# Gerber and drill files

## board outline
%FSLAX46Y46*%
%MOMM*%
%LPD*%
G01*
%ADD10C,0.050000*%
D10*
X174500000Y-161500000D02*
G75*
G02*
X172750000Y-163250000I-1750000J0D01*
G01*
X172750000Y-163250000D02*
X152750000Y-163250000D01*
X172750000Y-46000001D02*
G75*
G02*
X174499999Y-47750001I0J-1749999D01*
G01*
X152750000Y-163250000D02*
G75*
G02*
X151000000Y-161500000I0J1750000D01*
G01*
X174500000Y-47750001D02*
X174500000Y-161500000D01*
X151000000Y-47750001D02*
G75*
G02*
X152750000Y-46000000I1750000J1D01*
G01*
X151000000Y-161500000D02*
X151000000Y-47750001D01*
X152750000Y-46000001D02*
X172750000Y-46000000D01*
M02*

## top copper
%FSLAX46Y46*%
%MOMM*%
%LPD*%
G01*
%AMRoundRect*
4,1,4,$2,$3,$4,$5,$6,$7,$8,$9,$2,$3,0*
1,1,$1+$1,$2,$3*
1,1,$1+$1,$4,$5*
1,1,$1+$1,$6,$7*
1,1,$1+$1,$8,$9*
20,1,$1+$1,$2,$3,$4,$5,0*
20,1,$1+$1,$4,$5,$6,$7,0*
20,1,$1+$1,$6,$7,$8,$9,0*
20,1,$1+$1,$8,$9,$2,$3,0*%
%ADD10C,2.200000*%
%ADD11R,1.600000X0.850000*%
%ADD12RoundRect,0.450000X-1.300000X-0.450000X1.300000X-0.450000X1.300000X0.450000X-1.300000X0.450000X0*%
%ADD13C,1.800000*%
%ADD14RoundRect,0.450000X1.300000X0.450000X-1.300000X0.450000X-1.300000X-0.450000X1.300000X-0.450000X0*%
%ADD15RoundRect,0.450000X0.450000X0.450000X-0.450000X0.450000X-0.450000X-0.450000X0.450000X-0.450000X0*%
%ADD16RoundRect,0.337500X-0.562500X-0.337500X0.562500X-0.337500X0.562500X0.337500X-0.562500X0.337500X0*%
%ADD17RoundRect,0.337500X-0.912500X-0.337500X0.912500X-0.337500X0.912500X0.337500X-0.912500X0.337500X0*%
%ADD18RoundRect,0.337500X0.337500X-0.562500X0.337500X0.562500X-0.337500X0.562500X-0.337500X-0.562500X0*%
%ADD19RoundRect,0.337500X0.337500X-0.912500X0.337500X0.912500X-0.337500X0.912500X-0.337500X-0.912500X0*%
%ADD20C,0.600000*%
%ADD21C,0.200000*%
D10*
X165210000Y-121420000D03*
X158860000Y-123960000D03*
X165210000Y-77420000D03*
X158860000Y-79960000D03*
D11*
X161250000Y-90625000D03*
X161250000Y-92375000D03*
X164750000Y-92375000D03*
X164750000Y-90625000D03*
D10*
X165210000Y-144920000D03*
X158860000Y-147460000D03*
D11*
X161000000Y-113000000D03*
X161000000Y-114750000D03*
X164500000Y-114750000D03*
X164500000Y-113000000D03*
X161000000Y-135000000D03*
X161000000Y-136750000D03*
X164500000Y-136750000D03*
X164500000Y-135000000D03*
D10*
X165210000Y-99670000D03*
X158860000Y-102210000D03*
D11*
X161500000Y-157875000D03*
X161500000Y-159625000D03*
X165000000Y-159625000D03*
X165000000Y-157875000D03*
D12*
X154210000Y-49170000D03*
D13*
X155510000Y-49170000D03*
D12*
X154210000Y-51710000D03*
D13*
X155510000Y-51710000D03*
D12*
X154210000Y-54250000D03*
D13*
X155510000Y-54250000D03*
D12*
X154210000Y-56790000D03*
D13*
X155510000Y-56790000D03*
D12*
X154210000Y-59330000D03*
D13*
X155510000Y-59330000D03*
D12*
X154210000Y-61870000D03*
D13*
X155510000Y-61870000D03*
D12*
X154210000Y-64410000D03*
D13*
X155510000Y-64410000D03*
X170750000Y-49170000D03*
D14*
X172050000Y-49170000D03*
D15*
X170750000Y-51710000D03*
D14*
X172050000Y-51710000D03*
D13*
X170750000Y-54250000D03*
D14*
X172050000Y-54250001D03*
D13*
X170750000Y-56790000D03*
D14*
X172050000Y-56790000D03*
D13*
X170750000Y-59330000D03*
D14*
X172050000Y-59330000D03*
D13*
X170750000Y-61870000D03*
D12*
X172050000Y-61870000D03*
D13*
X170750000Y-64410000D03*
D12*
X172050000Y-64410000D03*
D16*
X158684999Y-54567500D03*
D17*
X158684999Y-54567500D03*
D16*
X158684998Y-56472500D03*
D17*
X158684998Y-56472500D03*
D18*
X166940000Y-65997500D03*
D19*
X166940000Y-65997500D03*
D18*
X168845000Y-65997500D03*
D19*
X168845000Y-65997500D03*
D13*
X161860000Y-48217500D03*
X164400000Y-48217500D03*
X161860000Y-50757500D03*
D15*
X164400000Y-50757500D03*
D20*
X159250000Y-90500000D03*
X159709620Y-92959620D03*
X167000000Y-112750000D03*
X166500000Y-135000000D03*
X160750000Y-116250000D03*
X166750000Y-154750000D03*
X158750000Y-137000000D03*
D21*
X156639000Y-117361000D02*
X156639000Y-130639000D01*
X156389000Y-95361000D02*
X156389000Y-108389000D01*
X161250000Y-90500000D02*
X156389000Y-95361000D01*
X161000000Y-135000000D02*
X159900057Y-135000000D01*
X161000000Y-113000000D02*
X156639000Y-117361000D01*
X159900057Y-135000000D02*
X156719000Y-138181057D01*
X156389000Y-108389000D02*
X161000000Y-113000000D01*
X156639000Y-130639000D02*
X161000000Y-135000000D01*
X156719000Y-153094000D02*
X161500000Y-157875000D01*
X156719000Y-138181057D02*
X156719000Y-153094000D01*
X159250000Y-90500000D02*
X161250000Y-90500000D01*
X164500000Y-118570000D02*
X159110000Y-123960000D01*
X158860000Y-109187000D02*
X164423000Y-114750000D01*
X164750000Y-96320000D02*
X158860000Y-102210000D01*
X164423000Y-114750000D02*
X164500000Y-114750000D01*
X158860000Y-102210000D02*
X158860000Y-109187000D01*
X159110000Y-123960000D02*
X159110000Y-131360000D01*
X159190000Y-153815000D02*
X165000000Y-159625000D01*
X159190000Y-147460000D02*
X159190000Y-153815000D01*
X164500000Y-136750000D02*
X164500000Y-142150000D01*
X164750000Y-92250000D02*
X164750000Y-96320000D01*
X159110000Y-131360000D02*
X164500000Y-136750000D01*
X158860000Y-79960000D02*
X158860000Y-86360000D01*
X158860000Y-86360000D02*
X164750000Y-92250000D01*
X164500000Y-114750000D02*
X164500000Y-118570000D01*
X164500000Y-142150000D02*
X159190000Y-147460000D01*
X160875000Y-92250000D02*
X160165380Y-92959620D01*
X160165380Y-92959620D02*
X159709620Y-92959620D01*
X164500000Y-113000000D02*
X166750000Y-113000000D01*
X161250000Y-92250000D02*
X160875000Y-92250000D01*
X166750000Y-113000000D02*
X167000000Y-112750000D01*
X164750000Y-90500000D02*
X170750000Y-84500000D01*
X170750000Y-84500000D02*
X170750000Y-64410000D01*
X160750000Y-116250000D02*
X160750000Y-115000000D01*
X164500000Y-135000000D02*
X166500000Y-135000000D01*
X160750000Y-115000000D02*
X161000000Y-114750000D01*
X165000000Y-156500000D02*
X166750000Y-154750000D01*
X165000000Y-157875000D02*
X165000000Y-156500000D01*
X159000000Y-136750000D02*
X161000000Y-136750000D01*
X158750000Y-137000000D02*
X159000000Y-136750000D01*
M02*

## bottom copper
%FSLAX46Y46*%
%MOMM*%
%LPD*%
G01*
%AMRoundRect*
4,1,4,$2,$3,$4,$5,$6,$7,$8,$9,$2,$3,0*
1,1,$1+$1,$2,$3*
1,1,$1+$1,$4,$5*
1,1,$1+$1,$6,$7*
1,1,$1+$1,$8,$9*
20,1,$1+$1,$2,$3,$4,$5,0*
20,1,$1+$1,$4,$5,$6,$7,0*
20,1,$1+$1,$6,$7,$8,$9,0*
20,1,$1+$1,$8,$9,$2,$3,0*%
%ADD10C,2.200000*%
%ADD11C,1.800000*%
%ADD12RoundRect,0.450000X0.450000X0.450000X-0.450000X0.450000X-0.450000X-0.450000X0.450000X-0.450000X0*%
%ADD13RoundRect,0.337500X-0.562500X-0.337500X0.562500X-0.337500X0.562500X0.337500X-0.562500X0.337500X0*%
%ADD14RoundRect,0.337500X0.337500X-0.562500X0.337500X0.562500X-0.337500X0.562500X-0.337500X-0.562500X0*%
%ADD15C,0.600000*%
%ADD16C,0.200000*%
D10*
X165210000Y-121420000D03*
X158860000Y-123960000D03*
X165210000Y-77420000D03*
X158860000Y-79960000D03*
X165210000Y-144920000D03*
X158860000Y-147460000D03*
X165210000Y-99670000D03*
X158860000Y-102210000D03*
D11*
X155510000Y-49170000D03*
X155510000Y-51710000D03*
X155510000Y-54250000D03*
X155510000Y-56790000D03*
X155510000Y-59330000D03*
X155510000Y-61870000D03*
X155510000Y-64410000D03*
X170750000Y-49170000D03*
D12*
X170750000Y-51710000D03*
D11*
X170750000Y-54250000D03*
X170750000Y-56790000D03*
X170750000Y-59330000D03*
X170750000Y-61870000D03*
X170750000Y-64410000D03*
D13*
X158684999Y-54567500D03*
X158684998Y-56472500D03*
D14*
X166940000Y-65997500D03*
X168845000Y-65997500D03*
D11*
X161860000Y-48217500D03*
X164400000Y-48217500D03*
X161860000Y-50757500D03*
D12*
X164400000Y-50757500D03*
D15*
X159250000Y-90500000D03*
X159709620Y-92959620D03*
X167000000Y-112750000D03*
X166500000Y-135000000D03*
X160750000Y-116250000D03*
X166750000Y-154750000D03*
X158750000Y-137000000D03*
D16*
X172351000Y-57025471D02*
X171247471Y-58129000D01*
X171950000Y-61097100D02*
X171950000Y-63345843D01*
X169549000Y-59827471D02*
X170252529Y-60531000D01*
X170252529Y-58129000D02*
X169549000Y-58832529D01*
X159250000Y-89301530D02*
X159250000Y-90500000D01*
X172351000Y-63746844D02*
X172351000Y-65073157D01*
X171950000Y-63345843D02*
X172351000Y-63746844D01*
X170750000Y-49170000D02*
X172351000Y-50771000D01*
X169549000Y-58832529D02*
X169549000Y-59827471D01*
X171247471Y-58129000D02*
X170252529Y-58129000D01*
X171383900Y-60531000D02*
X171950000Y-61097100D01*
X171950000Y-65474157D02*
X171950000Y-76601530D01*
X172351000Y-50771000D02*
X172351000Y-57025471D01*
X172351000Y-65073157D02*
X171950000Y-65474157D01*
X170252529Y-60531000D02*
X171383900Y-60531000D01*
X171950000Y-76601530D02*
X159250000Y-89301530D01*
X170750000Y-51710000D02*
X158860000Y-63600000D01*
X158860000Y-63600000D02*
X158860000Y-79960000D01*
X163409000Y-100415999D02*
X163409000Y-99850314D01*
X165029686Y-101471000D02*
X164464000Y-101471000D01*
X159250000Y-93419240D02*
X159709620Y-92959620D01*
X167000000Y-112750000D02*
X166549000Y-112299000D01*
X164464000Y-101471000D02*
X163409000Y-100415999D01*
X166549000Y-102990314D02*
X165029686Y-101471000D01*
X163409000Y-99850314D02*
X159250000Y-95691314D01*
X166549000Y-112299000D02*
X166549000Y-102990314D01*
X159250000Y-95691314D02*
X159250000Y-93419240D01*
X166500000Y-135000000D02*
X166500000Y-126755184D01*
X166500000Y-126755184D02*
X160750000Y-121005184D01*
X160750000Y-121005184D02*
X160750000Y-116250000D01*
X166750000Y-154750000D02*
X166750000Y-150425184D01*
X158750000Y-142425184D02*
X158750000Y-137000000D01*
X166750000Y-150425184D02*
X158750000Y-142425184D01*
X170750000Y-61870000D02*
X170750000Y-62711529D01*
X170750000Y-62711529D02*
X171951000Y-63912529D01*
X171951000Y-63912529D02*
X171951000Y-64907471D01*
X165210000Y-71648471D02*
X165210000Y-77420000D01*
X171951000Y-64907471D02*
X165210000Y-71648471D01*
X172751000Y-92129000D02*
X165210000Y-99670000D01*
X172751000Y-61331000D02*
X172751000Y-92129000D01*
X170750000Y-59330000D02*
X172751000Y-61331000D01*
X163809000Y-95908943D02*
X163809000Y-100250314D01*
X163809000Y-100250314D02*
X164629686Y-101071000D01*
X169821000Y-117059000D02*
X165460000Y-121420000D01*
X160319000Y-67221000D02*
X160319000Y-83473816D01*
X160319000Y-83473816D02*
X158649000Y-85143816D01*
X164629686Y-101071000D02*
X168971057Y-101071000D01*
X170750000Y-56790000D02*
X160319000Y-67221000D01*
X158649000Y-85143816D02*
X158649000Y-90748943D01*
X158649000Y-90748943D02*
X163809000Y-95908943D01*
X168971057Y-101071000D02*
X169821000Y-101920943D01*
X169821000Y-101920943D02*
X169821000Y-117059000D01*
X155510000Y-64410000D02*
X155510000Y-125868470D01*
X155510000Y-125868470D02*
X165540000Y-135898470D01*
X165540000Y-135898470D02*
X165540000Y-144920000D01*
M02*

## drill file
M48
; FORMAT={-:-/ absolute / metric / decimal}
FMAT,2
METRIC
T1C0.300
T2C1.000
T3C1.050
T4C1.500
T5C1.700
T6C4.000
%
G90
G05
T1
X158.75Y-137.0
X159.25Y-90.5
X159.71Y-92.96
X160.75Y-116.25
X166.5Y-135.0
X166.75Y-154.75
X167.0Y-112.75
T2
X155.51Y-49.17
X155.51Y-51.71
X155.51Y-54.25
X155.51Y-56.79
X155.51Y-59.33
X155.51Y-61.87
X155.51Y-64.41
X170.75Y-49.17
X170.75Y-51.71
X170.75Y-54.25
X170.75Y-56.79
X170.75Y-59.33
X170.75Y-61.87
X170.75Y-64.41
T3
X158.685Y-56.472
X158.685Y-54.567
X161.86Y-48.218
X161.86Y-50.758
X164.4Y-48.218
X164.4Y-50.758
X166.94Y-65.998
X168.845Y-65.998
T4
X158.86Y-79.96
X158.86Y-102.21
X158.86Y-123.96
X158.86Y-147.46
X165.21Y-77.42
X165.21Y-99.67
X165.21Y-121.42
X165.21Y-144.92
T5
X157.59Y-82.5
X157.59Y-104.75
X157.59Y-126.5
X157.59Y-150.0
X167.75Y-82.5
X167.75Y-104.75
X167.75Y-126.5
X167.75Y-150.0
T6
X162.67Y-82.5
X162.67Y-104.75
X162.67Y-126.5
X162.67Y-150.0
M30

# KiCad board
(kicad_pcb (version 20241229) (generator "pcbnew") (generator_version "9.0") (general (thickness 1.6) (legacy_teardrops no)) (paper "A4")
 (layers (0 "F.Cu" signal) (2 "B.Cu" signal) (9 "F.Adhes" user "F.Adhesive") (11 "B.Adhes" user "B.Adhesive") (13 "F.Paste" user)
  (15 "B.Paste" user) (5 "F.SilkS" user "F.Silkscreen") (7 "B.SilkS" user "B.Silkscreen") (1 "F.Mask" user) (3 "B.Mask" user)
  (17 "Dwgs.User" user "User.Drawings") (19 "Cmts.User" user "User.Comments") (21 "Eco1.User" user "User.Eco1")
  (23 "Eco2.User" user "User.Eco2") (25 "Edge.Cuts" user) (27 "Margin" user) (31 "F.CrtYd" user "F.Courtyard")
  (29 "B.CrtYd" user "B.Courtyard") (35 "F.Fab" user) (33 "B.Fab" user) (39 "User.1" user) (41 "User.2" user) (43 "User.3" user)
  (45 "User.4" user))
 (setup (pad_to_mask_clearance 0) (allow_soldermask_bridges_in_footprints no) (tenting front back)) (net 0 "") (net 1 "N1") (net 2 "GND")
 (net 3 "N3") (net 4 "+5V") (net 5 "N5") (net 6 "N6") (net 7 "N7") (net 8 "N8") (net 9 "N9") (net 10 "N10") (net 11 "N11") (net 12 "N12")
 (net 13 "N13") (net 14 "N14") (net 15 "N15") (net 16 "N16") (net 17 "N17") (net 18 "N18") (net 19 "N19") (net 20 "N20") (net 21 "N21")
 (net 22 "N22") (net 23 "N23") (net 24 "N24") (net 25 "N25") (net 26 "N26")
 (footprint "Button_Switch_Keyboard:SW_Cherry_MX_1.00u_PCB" (layer "F.Cu") (at 165.21 121.42)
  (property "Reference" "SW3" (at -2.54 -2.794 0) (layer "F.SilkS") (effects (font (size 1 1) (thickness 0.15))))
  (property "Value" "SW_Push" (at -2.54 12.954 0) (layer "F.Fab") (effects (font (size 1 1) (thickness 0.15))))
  (pad "" np_thru_hole circle (at -7.62 5.08) (size 1.7 1.7) (drill 1.7) (layers "*.Cu" "*.Mask"))
  (pad "" np_thru_hole circle (at -2.54 5.08) (size 4 4) (drill 4) (layers "*.Cu" "*.Mask"))
  (pad "" np_thru_hole circle (at 2.54 5.08) (size 1.7 1.7) (drill 1.7) (layers "*.Cu" "*.Mask"))
  (pad "1" thru_hole circle (at 0 0) (size 2.2 2.2) (drill 1.5) (layers "*.Cu" "*.Mask") (remove_unused_layers no) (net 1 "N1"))
  (pad "2" thru_hole circle (at -6.35 2.54) (size 2.2 2.2) (drill 1.5) (layers "*.Cu" "*.Mask") (remove_unused_layers no) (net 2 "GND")))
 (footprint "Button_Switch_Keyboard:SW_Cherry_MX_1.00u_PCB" (layer "F.Cu") (at 165.21 77.42)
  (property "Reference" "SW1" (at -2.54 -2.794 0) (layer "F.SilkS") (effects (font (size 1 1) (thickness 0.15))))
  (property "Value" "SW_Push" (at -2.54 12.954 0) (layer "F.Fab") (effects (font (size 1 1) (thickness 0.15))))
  (pad "" np_thru_hole circle (at -7.62 5.08) (size 1.7 1.7) (drill 1.7) (layers "*.Cu" "*.Mask"))
  (pad "" np_thru_hole circle (at -2.54 5.08) (size 4 4) (drill 4) (layers "*.Cu" "*.Mask"))
  (pad "" np_thru_hole circle (at 2.54 5.08) (size 1.7 1.7) (drill 1.7) (layers "*.Cu" "*.Mask"))
  (pad "1" thru_hole circle (at 0 0) (size 2.2 2.2) (drill 1.5) (layers "*.Cu" "*.Mask") (remove_unused_layers no) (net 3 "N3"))
  (pad "2" thru_hole circle (at -6.35 2.54) (size 2.2 2.2) (drill 1.5) (layers "*.Cu" "*.Mask") (remove_unused_layers no) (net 2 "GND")))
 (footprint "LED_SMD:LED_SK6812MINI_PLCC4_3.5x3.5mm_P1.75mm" (layer "F.Cu") (at 163 91.5)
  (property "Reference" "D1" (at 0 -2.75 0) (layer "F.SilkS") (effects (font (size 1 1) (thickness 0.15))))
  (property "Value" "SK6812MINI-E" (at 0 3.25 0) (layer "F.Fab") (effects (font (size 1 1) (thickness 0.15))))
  (pad "1" smd rect (at -1.75 -0.875) (size 1.6 0.85) (layers "F.Cu" "F.Mask" "F.Paste") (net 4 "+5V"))
  (pad "2" smd rect (at -1.75 0.875) (size 1.6 0.85) (layers "F.Cu" "F.Mask" "F.Paste") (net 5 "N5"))
  (pad "3" smd rect (at 1.75 0.875) (size 1.6 0.85) (layers "F.Cu" "F.Mask" "F.Paste") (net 2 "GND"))
  (pad "4" smd rect (at 1.75 -0.875) (size 1.6 0.85) (layers "F.Cu" "F.Mask" "F.Paste") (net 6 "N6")))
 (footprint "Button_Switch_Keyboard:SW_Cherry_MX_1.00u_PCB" (layer "F.Cu") (at 165.21 144.92)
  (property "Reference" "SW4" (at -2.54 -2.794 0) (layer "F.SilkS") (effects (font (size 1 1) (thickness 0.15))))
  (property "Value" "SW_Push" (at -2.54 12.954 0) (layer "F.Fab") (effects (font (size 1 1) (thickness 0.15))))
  (pad "" np_thru_hole circle (at -7.62 5.08) (size 1.7 1.7) (drill 1.7) (layers "*.Cu" "*.Mask"))
  (pad "" np_thru_hole circle (at -2.54 5.08) (size 4 4) (drill 4) (layers "*.Cu" "*.Mask"))
  (pad "" np_thru_hole circle (at 2.54 5.08) (size 1.7 1.7) (drill 1.7) (layers "*.Cu" "*.Mask"))
  (pad "1" thru_hole circle (at 0 0) (size 2.2 2.2) (drill 1.5) (layers "*.Cu" "*.Mask") (remove_unused_layers no) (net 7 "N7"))
  (pad "2" thru_hole circle (at -6.35 2.54) (size 2.2 2.2) (drill 1.5) (layers "*.Cu" "*.Mask") (remove_unused_layers no) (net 2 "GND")))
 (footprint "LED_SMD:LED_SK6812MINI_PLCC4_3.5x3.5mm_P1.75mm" (layer "F.Cu") (at 162.75 113.875)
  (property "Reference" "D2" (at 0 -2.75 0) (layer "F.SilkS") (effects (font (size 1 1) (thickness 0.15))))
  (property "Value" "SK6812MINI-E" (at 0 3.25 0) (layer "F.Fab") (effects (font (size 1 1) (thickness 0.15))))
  (pad "1" smd rect (at -1.75 -0.875) (size 1.6 0.85) (layers "F.Cu" "F.Mask" "F.Paste") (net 4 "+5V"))
  (pad "2" smd rect (at -1.75 0.875) (size 1.6 0.85) (layers "F.Cu" "F.Mask" "F.Paste") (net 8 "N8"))
  (pad "3" smd rect (at 1.75 0.875) (size 1.6 0.85) (layers "F.Cu" "F.Mask" "F.Paste") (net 2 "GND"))
  (pad "4" smd rect (at 1.75 -0.875) (size 1.6 0.85) (layers "F.Cu" "F.Mask" "F.Paste") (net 5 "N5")))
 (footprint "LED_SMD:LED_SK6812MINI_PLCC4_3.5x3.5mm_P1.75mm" (layer "F.Cu") (at 162.75 135.875)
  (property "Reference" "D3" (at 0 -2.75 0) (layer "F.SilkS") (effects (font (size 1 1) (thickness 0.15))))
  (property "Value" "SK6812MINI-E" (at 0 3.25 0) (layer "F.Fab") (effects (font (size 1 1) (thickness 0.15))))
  (pad "1" smd rect (at -1.75 -0.875) (size 1.6 0.85) (layers "F.Cu" "F.Mask" "F.Paste") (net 4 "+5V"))
  (pad "2" smd rect (at -1.75 0.875) (size 1.6 0.85) (layers "F.Cu" "F.Mask" "F.Paste") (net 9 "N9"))
  (pad "3" smd rect (at 1.75 0.875) (size 1.6 0.85) (layers "F.Cu" "F.Mask" "F.Paste") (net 2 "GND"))
  (pad "4" smd rect (at 1.75 -0.875) (size 1.6 0.85) (layers "F.Cu" "F.Mask" "F.Paste") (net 8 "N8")))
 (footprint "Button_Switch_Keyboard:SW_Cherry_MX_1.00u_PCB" (layer "F.Cu") (at 165.21 99.67)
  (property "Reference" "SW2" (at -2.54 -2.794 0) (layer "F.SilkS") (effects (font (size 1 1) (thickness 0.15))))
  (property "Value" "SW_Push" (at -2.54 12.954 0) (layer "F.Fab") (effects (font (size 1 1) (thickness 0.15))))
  (pad "" np_thru_hole circle (at -7.62 5.08) (size 1.7 1.7) (drill 1.7) (layers "*.Cu" "*.Mask"))
  (pad "" np_thru_hole circle (at -2.54 5.08) (size 4 4) (drill 4) (layers "*.Cu" "*.Mask"))
  (pad "" np_thru_hole circle (at 2.54 5.08) (size 1.7 1.7) (drill 1.7) (layers "*.Cu" "*.Mask"))
  (pad "1" thru_hole circle (at 0 0) (size 2.2 2.2) (drill 1.5) (layers "*.Cu" "*.Mask") (remove_unused_layers no) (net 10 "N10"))
  (pad "2" thru_hole circle (at -6.35 2.54) (size 2.2 2.2) (drill 1.5) (layers "*.Cu" "*.Mask") (remove_unused_layers no) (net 2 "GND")))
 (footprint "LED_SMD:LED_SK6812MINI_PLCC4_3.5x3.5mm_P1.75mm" (layer "F.Cu") (at 163.25 158.75)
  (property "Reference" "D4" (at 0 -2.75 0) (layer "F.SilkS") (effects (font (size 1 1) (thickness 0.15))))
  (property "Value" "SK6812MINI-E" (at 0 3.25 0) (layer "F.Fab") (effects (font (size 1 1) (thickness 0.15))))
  (pad "1" smd rect (at -1.75 -0.875) (size 1.6 0.85) (layers "F.Cu" "F.Mask" "F.Paste") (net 4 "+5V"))
  (pad "2" smd rect (at -1.75 0.875) (size 1.6 0.85) (layers "F.Cu" "F.Mask" "F.Paste") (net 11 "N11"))
  (pad "3" smd rect (at 1.75 0.875) (size 1.6 0.85) (layers "F.Cu" "F.Mask" "F.Paste") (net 2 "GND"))
  (pad "4" smd rect (at 1.75 -0.875) (size 1.6 0.85) (layers "F.Cu" "F.Mask" "F.Paste") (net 9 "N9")))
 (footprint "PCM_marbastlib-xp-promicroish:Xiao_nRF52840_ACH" (layer "F.Cu") (at 163.13 56.79)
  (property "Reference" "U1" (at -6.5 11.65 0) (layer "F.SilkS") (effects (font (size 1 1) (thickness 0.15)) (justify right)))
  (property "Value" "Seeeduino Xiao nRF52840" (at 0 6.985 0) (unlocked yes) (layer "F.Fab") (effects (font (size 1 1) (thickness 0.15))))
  (pad "1" smd roundrect (at -8.92 -7.62) (size 3.5 1.8) (layers "F.Cu" "F.Mask") (roundrect_rratio 0.25) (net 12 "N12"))
  (pad "1" thru_hole circle (at -7.62 -7.62) (size 1.8 1.8) (drill 1) (layers "*.Cu" "*.Mask") (remove_unused_layers no) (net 12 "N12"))
  (pad "2" smd roundrect (at -8.92 -5.08) (size 3.5 1.8) (layers "F.Cu" "F.Mask") (roundrect_rratio 0.25) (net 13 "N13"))
  (pad "2" thru_hole circle (at -7.62 -5.08) (size 1.8 1.8) (drill 1) (layers "*.Cu" "*.Mask") (remove_unused_layers no) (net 13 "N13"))
  (pad "3" smd roundrect (at -8.92 -2.54) (size 3.5 1.8) (layers "F.Cu" "F.Mask") (roundrect_rratio 0.25) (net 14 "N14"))
  (pad "3" thru_hole circle (at -7.62 -2.54) (size 1.8 1.8) (drill 1) (layers "*.Cu" "*.Mask") (remove_unused_layers no) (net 14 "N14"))
  (pad "4" smd roundrect (at -8.92 0) (size 3.5 1.8) (layers "F.Cu" "F.Mask") (roundrect_rratio 0.25) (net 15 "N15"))
  (pad "4" thru_hole circle (at -7.62 0) (size 1.8 1.8) (drill 1) (layers "*.Cu" "*.Mask") (remove_unused_layers no) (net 15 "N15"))
  (pad "5" smd roundrect (at -8.92 2.54) (size 3.5 1.8) (layers "F.Cu" "F.Mask") (roundrect_rratio 0.25) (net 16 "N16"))
  (pad "5" thru_hole circle (at -7.62 2.54) (size 1.8 1.8) (drill 1) (layers "*.Cu" "*.Mask") (remove_unused_layers no) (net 16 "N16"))
  (pad "6" smd roundrect (at -8.92 5.08) (size 3.5 1.8) (layers "F.Cu" "F.Mask") (roundrect_rratio 0.25) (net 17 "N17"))
  (pad "6" thru_hole circle (at -7.62 5.08) (size 1.8 1.8) (drill 1) (layers "*.Cu" "*.Mask") (remove_unused_layers no) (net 17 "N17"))
  (pad "7" smd roundrect (at -8.92 7.62) (size 3.5 1.8) (layers "F.Cu" "F.Mask") (roundrect_rratio 0.25) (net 7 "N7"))
  (pad "7" thru_hole circle (at -7.62 7.62) (size 1.8 1.8) (drill 1) (layers "*.Cu" "*.Mask") (remove_unused_layers no) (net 7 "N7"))
  (pad "8" thru_hole circle (at 7.62 -7.62 180) (size 1.8 1.8) (drill 1) (layers "*.Cu" "*.Mask") (remove_unused_layers no) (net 4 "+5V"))
  (pad "8" smd roundrect (at 8.92 -7.62 180) (size 3.5 1.8) (layers "F.Cu" "F.Mask") (roundrect_rratio 0.25) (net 4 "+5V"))
  (pad "9" thru_hole roundrect (at 7.62 -5.08 180) (size 1.8 1.8) (drill 1) (layers "*.Cu" "*.Mask") (remove_unused_layers no)
   (roundrect_rratio 0.25) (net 2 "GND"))
  (pad "9" smd roundrect (at 8.92 -5.08 180) (size 3.5 1.8) (layers "F.Cu" "F.Mask") (roundrect_rratio 0.25) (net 2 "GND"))
  (pad "10" thru_hole circle (at 7.62 -2.54 180) (size 1.8 1.8) (drill 1) (layers "*.Cu" "*.Mask") (remove_unused_layers no) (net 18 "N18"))
  (pad "10" smd roundrect (at 8.92 -2.539999 180) (size 3.5 1.8) (layers "F.Cu" "F.Mask") (roundrect_rratio 0.25) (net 18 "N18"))
  (pad "11" thru_hole circle (at 7.62 0 180) (size 1.8 1.8) (drill 1) (layers "*.Cu" "*.Mask") (remove_unused_layers no) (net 1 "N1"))
  (pad "11" smd roundrect (at 8.92 0 180) (size 3.5 1.8) (layers "F.Cu" "F.Mask") (roundrect_rratio 0.25) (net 1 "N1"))
  (pad "12" thru_hole circle (at 7.62 2.54 180) (size 1.8 1.8) (drill 1) (layers "*.Cu" "*.Mask") (remove_unused_layers no) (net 10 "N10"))
  (pad "12" smd roundrect (at 8.92 2.54 180) (size 3.5 1.8) (layers "F.Cu" "F.Mask") (roundrect_rratio 0.25) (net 10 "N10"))
  (pad "13" thru_hole circle (at 7.62 5.08) (size 1.8 1.8) (drill 1) (layers "*.Cu" "*.Mask") (remove_unused_layers no) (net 3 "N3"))
  (pad "13" smd roundrect (at 8.92 5.08) (size 3.5 1.8) (layers "F.Cu" "F.Mask") (roundrect_rratio 0.25) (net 3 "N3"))
  (pad "14" thru_hole circle (at 7.62 7.62) (size 1.8 1.8) (drill 1) (layers "*.Cu" "*.Mask") (remove_unused_layers no) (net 6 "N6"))
  (pad "14" smd roundrect (at 8.92 7.62) (size 3.5 1.8) (layers "F.Cu" "F.Mask") (roundrect_rratio 0.25) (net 6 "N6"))
  (pad "15" thru_hole roundrect (at -4.445001 -2.2225) (size 1.8 1.35) (drill 1.05) (layers "*.Cu" "*.Mask") (remove_unused_layers no)
   (roundrect_rratio 0.25) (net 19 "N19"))
  (pad "15" smd roundrect (at -4.445001 -2.2225) (size 2.5 1.35) (layers "F.Cu" "F.Mask") (roundrect_rratio 0.25) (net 19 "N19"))
  (pad "16" thru_hole roundrect (at -4.445002 -0.3175) (size 1.8 1.35) (drill 1.05) (layers "*.Cu" "*.Mask") (remove_unused_layers no)
   (roundrect_rratio 0.25) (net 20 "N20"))
  (pad "16" smd roundrect (at -4.445002 -0.3175) (size 2.5 1.35) (layers "F.Cu" "F.Mask") (roundrect_rratio 0.25) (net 20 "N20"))
  (pad "17" thru_hole roundrect (at 3.81 9.2075 90) (size 1.8 1.35) (drill 1.05) (layers "*.Cu" "*.Mask") (remove_unused_layers no)
   (roundrect_rratio 0.25) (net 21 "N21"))
  (pad "17" smd roundrect (at 3.81 9.2075 90) (size 2.5 1.35) (layers "F.Cu" "F.Mask") (roundrect_rratio 0.25) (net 21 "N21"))
  (pad "18" thru_hole roundrect (at 5.715 9.2075 90) (size 1.8 1.35) (drill 1.05) (layers "*.Cu" "*.Mask") (remove_unused_layers no)
   (roundrect_rratio 0.25) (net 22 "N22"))
  (pad "18" smd roundrect (at 5.715 9.2075 90) (size 2.5 1.35) (layers "F.Cu" "F.Mask") (roundrect_rratio 0.25) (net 22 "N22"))
  (pad "19" thru_hole circle (at -1.27 -8.5725 180) (size 1.8 1.8) (drill 1.05) (layers "*.Cu" "*.Mask") (remove_unused_layers no)
   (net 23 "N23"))
  (pad "20" thru_hole circle (at 1.27 -8.5725 180) (size 1.8 1.8) (drill 1.05) (layers "*.Cu" "*.Mask") (remove_unused_layers no)
   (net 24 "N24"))
  (pad "21" thru_hole circle (at -1.27 -6.0325 180) (size 1.8 1.8) (drill 1.05) (layers "*.Cu" "*.Mask") (remove_unused_layers no)
   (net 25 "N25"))
  (pad "22" thru_hole roundrect (at 1.27 -6.0325 180) (size 1.8 1.8) (drill 1.05) (layers "*.Cu" "*.Mask") (remove_unused_layers no)
   (roundrect_rratio 0.25) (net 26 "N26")))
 (gr_arc (start 174.5 161.5) (mid 173.987437 162.737437) (end 172.75 163.25) (stroke (width 0.05) (type default)) (layer "Edge.Cuts"))
 (gr_line (start 172.75 163.25) (end 152.75 163.25) (stroke (width 0.05) (type default)) (layer "Edge.Cuts"))
 (gr_arc (start 172.75 46.000001) (mid 173.987437 46.512564) (end 174.5 47.750001) (stroke (width 0.05) (type default)) (layer "Edge.Cuts"))
 (gr_arc (start 152.75 163.25) (mid 151.512563 162.737437) (end 151 161.5) (stroke (width 0.05) (type default)) (layer "Edge.Cuts"))
 (gr_line (start 174.5 47.750001) (end 174.5 161.5) (stroke (width 0.05) (type default)) (layer "Edge.Cuts"))
 (gr_arc (start 151 47.750001) (mid 151.512563 46.512564) (end 152.75 46.000001) (stroke (width 0.05) (type default)) (layer "Edge.Cuts"))
 (gr_line (start 151 161.5) (end 151 47.750001) (stroke (width 0.05) (type default)) (layer "Edge.Cuts"))
 (gr_line (start 152.75 46.000001) (end 172.75 46) (stroke (width 0.05) (type default)) (layer "Edge.Cuts"))
 (segment (start 156.639 117.361) (end 156.639 130.639) (width 0.2) (layer "F.Cu") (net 4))
 (segment (start 156.389 95.361) (end 156.389 108.389) (width 0.2) (layer "F.Cu") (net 4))
 (segment (start 161.25 90.5) (end 156.389 95.361) (width 0.2) (layer "F.Cu") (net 4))
 (segment (start 161 135) (end 159.900057 135) (width 0.2) (layer "F.Cu") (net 4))
 (segment (start 161 113) (end 156.639 117.361) (width 0.2) (layer "F.Cu") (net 4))
 (segment (start 159.900057 135) (end 156.719 138.181057) (width 0.2) (layer "F.Cu") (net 4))
 (segment (start 156.389 108.389) (end 161 113) (width 0.2) (layer "F.Cu") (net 4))
 (segment (start 156.639 130.639) (end 161 135) (width 0.2) (layer "F.Cu") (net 4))
 (segment (start 156.719 153.094) (end 161.5 157.875) (width 0.2) (layer "F.Cu") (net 4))
 (segment (start 156.719 138.181057) (end 156.719 153.094) (width 0.2) (layer "F.Cu") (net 4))
 (segment (start 159.25 90.5) (end 161.25 90.5) (width 0.2) (layer "F.Cu") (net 4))
 (via (at 159.25 90.5) (size 0.6) (drill 0.3) (layers "F.Cu" "B.Cu") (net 4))
 (segment (start 172.351 57.025471) (end 171.247471 58.129) (width 0.2) (layer "B.Cu") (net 4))
 (segment (start 171.95 61.0971) (end 171.95 63.345843) (width 0.2) (layer "B.Cu") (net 4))
 (segment (start 169.549 59.827471) (end 170.252529 60.531) (width 0.2) (layer "B.Cu") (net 4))
 (segment (start 170.252529 58.129) (end 169.549 58.832529) (width 0.2) (layer "B.Cu") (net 4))
 (segment (start 159.25 89.30153) (end 159.25 90.5) (width 0.2) (layer "B.Cu") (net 4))
 (segment (start 172.351 63.746844) (end 172.351 65.073157) (width 0.2) (layer "B.Cu") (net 4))
 (segment (start 171.95 63.345843) (end 172.351 63.746844) (width 0.2) (layer "B.Cu") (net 4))
 (segment (start 170.75 49.17) (end 172.351 50.771) (width 0.2) (layer "B.Cu") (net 4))
 (segment (start 169.549 58.832529) (end 169.549 59.827471) (width 0.2) (layer "B.Cu") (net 4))
 (segment (start 171.247471 58.129) (end 170.252529 58.129) (width 0.2) (layer "B.Cu") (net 4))
 (segment (start 171.3839 60.531) (end 171.95 61.0971) (width 0.2) (layer "B.Cu") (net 4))
 (segment (start 171.95 65.474157) (end 171.95 76.60153) (width 0.2) (layer "B.Cu") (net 4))
 (segment (start 172.351 50.771) (end 172.351 57.025471) (width 0.2) (layer "B.Cu") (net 4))
 (segment (start 172.351 65.073157) (end 171.95 65.474157) (width 0.2) (layer "B.Cu") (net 4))
 (segment (start 170.252529 60.531) (end 171.3839 60.531) (width 0.2) (layer "B.Cu") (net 4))
 (segment (start 171.95 76.60153) (end 159.25 89.30153) (width 0.2) (layer "B.Cu") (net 4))
 (segment (start 164.5 118.57) (end 159.11 123.96) (width 0.2) (layer "F.Cu") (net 2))
 (segment (start 158.86 109.187) (end 164.423 114.75) (width 0.2) (layer "F.Cu") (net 2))
 (segment (start 164.75 96.32) (end 158.86 102.21) (width 0.2) (layer "F.Cu") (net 2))
 (segment (start 164.423 114.75) (end 164.5 114.75) (width 0.2) (layer "F.Cu") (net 2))
 (segment (start 158.86 102.21) (end 158.86 109.187) (width 0.2) (layer "F.Cu") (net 2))
 (segment (start 159.11 123.96) (end 159.11 131.36) (width 0.2) (layer "F.Cu") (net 2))
 (segment (start 159.19 153.815) (end 165 159.625) (width 0.2) (layer "F.Cu") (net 2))
 (segment (start 159.19 147.46) (end 159.19 153.815) (width 0.2) (layer "F.Cu") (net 2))
 (segment (start 164.5 136.75) (end 164.5 142.15) (width 0.2) (layer "F.Cu") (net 2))
 (segment (start 164.75 92.25) (end 164.75 96.32) (width 0.2) (layer "F.Cu") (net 2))
 (segment (start 159.11 131.36) (end 164.5 136.75) (width 0.2) (layer "F.Cu") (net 2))
 (segment (start 158.86 79.96) (end 158.86 86.36) (width 0.2) (layer "F.Cu") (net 2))
 (segment (start 158.86 86.36) (end 164.75 92.25) (width 0.2) (layer "F.Cu") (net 2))
 (segment (start 164.5 114.75) (end 164.5 118.57) (width 0.2) (layer "F.Cu") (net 2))
 (segment (start 164.5 142.15) (end 159.19 147.46) (width 0.2) (layer "F.Cu") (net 2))
 (segment (start 170.75 51.71) (end 158.86 63.6) (width 0.2) (layer "B.Cu") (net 2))
 (segment (start 158.86 63.6) (end 158.86 79.96) (width 0.2) (layer "B.Cu") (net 2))
 (segment (start 160.875 92.25) (end 160.16538 92.95962) (width 0.2) (layer "F.Cu") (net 5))
 (segment (start 160.16538 92.95962) (end 159.70962 92.95962) (width 0.2) (layer "F.Cu") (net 5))
 (segment (start 164.5 113) (end 166.75 113) (width 0.2) (layer "F.Cu") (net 5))
 (segment (start 161.25 92.25) (end 160.875 92.25) (width 0.2) (layer "F.Cu") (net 5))
 (segment (start 166.75 113) (end 167 112.75) (width 0.2) (layer "F.Cu") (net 5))
 (via (at 159.70962 92.95962) (size 0.6) (drill 0.3) (layers "F.Cu" "B.Cu") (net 5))
 (via (at 167 112.75) (size 0.6) (drill 0.3) (layers "F.Cu" "B.Cu") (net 5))
 (segment (start 163.409 100.415999) (end 163.409 99.850314) (width 0.2) (layer "B.Cu") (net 5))
 (segment (start 165.029686 101.471) (end 164.464 101.471) (width 0.2) (layer "B.Cu") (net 5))
 (segment (start 159.25 93.41924) (end 159.70962 92.95962) (width 0.2) (layer "B.Cu") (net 5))
 (segment (start 167 112.75) (end 166.549 112.299) (width 0.2) (layer "B.Cu") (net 5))
 (segment (start 164.464 101.471) (end 163.409 100.415999) (width 0.2) (layer "B.Cu") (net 5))
 (segment (start 166.549 102.990314) (end 165.029686 101.471) (width 0.2) (layer "B.Cu") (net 5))
 (segment (start 163.409 99.850314) (end 159.25 95.691314) (width 0.2) (layer "B.Cu") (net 5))
 (segment (start 166.549 112.299) (end 166.549 102.990314) (width 0.2) (layer "B.Cu") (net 5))
 (segment (start 159.25 95.691314) (end 159.25 93.41924) (width 0.2) (layer "B.Cu") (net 5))
 (segment (start 164.75 90.5) (end 170.75 84.5) (width 0.2) (layer "F.Cu") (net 6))
 (segment (start 170.75 84.5) (end 170.75 64.41) (width 0.2) (layer "F.Cu") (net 6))
 (segment (start 160.75 116.25) (end 160.75 115) (width 0.2) (layer "F.Cu") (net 8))
 (segment (start 164.5 135) (end 166.5 135) (width 0.2) (layer "F.Cu") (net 8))
 (segment (start 160.75 115) (end 161 114.75) (width 0.2) (layer "F.Cu") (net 8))
 (via (at 166.5 135) (size 0.6) (drill 0.3) (layers "F.Cu" "B.Cu") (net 8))
 (via (at 160.75 116.25) (size 0.6) (drill 0.3) (layers "F.Cu" "B.Cu") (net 8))
 (segment (start 166.5 135) (end 166.5 126.755184) (width 0.2) (layer "B.Cu") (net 8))
 (segment (start 166.5 126.755184) (end 160.75 121.005184) (width 0.2) (layer "B.Cu") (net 8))
 (segment (start 160.75 121.005184) (end 160.75 116.25) (width 0.2) (layer "B.Cu") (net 8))
 (segment (start 165 156.5) (end 166.75 154.75) (width 0.2) (layer "F.Cu") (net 9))
 (segment (start 165 157.875) (end 165 156.5) (width 0.2) (layer "F.Cu") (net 9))
 (segment (start 159 136.75) (end 161 136.75) (width 0.2) (layer "F.Cu") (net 9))
 (segment (start 158.75 137) (end 159 136.75) (width 0.2) (layer "F.Cu") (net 9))
 (via (at 166.75 154.75) (size 0.6) (drill 0.3) (layers "F.Cu" "B.Cu") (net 9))
 (via (at 158.75 137) (size 0.6) (drill 0.3) (layers "F.Cu" "B.Cu") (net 9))
 (segment (start 166.75 154.75) (end 166.75 150.425184) (width 0.2) (layer "B.Cu") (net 9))
 (segment (start 158.75 142.425184) (end 158.75 137) (width 0.2) (layer "B.Cu") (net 9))
 (segment (start 166.75 150.425184) (end 158.75 142.425184) (width 0.2) (layer "B.Cu") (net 9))
 (segment (start 170.75 61.87) (end 170.75 62.711529) (width 0.2) (layer "B.Cu") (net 3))
 (segment (start 170.75 62.711529) (end 171.951 63.912529) (width 0.2) (layer "B.Cu") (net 3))
 (segment (start 171.951 63.912529) (end 171.951 64.907471) (width 0.2) (layer "B.Cu") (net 3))
 (segment (start 165.21 71.648471) (end 165.21 77.42) (width 0.2) (layer "B.Cu") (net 3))
 (segment (start 171.951 64.907471) (end 165.21 71.648471) (width 0.2) (layer "B.Cu") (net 3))
 (segment (start 172.751 92.129) (end 165.21 99.67) (width 0.2) (layer "B.Cu") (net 10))
 (segment (start 172.751 61.331) (end 172.751 92.129) (width 0.2) (layer "B.Cu") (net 10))
 (segment (start 170.75 59.33) (end 172.751 61.331) (width 0.2) (layer "B.Cu") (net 10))
 (segment (start 163.809 95.908943) (end 163.809 100.250314) (width 0.2) (layer "B.Cu") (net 1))
 (segment (start 163.809 100.250314) (end 164.629686 101.071) (width 0.2) (layer "B.Cu") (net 1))
 (segment (start 169.821 117.059) (end 165.46 121.42) (width 0.2) (layer "B.Cu") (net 1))
 (segment (start 160.319 67.221) (end 160.319 83.473816) (width 0.2) (layer "B.Cu") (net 1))
 (segment (start 160.319 83.473816) (end 158.649 85.143816) (width 0.2) (layer "B.Cu") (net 1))
 (segment (start 164.629686 101.071) (end 168.971057 101.071) (width 0.2) (layer "B.Cu") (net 1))
 (segment (start 170.75 56.79) (end 160.319 67.221) (width 0.2) (layer "B.Cu") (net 1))
 (segment (start 158.649 85.143816) (end 158.649 90.748943) (width 0.2) (layer "B.Cu") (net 1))
 (segment (start 158.649 90.748943) (end 163.809 95.908943) (width 0.2) (layer "B.Cu") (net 1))
 (segment (start 168.971057 101.071) (end 169.821 101.920943) (width 0.2) (layer "B.Cu") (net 1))
 (segment (start 169.821 101.920943) (end 169.821 117.059) (width 0.2) (layer "B.Cu") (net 1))
 (segment (start 155.51 64.41) (end 155.51 125.86847) (width 0.2) (layer "B.Cu") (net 7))
 (segment (start 155.51 125.86847) (end 165.54 135.89847) (width 0.2) (layer "B.Cu") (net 7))
 (segment (start 165.54 135.89847) (end 165.54 144.92) (width 0.2) (layer "B.Cu") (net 7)))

